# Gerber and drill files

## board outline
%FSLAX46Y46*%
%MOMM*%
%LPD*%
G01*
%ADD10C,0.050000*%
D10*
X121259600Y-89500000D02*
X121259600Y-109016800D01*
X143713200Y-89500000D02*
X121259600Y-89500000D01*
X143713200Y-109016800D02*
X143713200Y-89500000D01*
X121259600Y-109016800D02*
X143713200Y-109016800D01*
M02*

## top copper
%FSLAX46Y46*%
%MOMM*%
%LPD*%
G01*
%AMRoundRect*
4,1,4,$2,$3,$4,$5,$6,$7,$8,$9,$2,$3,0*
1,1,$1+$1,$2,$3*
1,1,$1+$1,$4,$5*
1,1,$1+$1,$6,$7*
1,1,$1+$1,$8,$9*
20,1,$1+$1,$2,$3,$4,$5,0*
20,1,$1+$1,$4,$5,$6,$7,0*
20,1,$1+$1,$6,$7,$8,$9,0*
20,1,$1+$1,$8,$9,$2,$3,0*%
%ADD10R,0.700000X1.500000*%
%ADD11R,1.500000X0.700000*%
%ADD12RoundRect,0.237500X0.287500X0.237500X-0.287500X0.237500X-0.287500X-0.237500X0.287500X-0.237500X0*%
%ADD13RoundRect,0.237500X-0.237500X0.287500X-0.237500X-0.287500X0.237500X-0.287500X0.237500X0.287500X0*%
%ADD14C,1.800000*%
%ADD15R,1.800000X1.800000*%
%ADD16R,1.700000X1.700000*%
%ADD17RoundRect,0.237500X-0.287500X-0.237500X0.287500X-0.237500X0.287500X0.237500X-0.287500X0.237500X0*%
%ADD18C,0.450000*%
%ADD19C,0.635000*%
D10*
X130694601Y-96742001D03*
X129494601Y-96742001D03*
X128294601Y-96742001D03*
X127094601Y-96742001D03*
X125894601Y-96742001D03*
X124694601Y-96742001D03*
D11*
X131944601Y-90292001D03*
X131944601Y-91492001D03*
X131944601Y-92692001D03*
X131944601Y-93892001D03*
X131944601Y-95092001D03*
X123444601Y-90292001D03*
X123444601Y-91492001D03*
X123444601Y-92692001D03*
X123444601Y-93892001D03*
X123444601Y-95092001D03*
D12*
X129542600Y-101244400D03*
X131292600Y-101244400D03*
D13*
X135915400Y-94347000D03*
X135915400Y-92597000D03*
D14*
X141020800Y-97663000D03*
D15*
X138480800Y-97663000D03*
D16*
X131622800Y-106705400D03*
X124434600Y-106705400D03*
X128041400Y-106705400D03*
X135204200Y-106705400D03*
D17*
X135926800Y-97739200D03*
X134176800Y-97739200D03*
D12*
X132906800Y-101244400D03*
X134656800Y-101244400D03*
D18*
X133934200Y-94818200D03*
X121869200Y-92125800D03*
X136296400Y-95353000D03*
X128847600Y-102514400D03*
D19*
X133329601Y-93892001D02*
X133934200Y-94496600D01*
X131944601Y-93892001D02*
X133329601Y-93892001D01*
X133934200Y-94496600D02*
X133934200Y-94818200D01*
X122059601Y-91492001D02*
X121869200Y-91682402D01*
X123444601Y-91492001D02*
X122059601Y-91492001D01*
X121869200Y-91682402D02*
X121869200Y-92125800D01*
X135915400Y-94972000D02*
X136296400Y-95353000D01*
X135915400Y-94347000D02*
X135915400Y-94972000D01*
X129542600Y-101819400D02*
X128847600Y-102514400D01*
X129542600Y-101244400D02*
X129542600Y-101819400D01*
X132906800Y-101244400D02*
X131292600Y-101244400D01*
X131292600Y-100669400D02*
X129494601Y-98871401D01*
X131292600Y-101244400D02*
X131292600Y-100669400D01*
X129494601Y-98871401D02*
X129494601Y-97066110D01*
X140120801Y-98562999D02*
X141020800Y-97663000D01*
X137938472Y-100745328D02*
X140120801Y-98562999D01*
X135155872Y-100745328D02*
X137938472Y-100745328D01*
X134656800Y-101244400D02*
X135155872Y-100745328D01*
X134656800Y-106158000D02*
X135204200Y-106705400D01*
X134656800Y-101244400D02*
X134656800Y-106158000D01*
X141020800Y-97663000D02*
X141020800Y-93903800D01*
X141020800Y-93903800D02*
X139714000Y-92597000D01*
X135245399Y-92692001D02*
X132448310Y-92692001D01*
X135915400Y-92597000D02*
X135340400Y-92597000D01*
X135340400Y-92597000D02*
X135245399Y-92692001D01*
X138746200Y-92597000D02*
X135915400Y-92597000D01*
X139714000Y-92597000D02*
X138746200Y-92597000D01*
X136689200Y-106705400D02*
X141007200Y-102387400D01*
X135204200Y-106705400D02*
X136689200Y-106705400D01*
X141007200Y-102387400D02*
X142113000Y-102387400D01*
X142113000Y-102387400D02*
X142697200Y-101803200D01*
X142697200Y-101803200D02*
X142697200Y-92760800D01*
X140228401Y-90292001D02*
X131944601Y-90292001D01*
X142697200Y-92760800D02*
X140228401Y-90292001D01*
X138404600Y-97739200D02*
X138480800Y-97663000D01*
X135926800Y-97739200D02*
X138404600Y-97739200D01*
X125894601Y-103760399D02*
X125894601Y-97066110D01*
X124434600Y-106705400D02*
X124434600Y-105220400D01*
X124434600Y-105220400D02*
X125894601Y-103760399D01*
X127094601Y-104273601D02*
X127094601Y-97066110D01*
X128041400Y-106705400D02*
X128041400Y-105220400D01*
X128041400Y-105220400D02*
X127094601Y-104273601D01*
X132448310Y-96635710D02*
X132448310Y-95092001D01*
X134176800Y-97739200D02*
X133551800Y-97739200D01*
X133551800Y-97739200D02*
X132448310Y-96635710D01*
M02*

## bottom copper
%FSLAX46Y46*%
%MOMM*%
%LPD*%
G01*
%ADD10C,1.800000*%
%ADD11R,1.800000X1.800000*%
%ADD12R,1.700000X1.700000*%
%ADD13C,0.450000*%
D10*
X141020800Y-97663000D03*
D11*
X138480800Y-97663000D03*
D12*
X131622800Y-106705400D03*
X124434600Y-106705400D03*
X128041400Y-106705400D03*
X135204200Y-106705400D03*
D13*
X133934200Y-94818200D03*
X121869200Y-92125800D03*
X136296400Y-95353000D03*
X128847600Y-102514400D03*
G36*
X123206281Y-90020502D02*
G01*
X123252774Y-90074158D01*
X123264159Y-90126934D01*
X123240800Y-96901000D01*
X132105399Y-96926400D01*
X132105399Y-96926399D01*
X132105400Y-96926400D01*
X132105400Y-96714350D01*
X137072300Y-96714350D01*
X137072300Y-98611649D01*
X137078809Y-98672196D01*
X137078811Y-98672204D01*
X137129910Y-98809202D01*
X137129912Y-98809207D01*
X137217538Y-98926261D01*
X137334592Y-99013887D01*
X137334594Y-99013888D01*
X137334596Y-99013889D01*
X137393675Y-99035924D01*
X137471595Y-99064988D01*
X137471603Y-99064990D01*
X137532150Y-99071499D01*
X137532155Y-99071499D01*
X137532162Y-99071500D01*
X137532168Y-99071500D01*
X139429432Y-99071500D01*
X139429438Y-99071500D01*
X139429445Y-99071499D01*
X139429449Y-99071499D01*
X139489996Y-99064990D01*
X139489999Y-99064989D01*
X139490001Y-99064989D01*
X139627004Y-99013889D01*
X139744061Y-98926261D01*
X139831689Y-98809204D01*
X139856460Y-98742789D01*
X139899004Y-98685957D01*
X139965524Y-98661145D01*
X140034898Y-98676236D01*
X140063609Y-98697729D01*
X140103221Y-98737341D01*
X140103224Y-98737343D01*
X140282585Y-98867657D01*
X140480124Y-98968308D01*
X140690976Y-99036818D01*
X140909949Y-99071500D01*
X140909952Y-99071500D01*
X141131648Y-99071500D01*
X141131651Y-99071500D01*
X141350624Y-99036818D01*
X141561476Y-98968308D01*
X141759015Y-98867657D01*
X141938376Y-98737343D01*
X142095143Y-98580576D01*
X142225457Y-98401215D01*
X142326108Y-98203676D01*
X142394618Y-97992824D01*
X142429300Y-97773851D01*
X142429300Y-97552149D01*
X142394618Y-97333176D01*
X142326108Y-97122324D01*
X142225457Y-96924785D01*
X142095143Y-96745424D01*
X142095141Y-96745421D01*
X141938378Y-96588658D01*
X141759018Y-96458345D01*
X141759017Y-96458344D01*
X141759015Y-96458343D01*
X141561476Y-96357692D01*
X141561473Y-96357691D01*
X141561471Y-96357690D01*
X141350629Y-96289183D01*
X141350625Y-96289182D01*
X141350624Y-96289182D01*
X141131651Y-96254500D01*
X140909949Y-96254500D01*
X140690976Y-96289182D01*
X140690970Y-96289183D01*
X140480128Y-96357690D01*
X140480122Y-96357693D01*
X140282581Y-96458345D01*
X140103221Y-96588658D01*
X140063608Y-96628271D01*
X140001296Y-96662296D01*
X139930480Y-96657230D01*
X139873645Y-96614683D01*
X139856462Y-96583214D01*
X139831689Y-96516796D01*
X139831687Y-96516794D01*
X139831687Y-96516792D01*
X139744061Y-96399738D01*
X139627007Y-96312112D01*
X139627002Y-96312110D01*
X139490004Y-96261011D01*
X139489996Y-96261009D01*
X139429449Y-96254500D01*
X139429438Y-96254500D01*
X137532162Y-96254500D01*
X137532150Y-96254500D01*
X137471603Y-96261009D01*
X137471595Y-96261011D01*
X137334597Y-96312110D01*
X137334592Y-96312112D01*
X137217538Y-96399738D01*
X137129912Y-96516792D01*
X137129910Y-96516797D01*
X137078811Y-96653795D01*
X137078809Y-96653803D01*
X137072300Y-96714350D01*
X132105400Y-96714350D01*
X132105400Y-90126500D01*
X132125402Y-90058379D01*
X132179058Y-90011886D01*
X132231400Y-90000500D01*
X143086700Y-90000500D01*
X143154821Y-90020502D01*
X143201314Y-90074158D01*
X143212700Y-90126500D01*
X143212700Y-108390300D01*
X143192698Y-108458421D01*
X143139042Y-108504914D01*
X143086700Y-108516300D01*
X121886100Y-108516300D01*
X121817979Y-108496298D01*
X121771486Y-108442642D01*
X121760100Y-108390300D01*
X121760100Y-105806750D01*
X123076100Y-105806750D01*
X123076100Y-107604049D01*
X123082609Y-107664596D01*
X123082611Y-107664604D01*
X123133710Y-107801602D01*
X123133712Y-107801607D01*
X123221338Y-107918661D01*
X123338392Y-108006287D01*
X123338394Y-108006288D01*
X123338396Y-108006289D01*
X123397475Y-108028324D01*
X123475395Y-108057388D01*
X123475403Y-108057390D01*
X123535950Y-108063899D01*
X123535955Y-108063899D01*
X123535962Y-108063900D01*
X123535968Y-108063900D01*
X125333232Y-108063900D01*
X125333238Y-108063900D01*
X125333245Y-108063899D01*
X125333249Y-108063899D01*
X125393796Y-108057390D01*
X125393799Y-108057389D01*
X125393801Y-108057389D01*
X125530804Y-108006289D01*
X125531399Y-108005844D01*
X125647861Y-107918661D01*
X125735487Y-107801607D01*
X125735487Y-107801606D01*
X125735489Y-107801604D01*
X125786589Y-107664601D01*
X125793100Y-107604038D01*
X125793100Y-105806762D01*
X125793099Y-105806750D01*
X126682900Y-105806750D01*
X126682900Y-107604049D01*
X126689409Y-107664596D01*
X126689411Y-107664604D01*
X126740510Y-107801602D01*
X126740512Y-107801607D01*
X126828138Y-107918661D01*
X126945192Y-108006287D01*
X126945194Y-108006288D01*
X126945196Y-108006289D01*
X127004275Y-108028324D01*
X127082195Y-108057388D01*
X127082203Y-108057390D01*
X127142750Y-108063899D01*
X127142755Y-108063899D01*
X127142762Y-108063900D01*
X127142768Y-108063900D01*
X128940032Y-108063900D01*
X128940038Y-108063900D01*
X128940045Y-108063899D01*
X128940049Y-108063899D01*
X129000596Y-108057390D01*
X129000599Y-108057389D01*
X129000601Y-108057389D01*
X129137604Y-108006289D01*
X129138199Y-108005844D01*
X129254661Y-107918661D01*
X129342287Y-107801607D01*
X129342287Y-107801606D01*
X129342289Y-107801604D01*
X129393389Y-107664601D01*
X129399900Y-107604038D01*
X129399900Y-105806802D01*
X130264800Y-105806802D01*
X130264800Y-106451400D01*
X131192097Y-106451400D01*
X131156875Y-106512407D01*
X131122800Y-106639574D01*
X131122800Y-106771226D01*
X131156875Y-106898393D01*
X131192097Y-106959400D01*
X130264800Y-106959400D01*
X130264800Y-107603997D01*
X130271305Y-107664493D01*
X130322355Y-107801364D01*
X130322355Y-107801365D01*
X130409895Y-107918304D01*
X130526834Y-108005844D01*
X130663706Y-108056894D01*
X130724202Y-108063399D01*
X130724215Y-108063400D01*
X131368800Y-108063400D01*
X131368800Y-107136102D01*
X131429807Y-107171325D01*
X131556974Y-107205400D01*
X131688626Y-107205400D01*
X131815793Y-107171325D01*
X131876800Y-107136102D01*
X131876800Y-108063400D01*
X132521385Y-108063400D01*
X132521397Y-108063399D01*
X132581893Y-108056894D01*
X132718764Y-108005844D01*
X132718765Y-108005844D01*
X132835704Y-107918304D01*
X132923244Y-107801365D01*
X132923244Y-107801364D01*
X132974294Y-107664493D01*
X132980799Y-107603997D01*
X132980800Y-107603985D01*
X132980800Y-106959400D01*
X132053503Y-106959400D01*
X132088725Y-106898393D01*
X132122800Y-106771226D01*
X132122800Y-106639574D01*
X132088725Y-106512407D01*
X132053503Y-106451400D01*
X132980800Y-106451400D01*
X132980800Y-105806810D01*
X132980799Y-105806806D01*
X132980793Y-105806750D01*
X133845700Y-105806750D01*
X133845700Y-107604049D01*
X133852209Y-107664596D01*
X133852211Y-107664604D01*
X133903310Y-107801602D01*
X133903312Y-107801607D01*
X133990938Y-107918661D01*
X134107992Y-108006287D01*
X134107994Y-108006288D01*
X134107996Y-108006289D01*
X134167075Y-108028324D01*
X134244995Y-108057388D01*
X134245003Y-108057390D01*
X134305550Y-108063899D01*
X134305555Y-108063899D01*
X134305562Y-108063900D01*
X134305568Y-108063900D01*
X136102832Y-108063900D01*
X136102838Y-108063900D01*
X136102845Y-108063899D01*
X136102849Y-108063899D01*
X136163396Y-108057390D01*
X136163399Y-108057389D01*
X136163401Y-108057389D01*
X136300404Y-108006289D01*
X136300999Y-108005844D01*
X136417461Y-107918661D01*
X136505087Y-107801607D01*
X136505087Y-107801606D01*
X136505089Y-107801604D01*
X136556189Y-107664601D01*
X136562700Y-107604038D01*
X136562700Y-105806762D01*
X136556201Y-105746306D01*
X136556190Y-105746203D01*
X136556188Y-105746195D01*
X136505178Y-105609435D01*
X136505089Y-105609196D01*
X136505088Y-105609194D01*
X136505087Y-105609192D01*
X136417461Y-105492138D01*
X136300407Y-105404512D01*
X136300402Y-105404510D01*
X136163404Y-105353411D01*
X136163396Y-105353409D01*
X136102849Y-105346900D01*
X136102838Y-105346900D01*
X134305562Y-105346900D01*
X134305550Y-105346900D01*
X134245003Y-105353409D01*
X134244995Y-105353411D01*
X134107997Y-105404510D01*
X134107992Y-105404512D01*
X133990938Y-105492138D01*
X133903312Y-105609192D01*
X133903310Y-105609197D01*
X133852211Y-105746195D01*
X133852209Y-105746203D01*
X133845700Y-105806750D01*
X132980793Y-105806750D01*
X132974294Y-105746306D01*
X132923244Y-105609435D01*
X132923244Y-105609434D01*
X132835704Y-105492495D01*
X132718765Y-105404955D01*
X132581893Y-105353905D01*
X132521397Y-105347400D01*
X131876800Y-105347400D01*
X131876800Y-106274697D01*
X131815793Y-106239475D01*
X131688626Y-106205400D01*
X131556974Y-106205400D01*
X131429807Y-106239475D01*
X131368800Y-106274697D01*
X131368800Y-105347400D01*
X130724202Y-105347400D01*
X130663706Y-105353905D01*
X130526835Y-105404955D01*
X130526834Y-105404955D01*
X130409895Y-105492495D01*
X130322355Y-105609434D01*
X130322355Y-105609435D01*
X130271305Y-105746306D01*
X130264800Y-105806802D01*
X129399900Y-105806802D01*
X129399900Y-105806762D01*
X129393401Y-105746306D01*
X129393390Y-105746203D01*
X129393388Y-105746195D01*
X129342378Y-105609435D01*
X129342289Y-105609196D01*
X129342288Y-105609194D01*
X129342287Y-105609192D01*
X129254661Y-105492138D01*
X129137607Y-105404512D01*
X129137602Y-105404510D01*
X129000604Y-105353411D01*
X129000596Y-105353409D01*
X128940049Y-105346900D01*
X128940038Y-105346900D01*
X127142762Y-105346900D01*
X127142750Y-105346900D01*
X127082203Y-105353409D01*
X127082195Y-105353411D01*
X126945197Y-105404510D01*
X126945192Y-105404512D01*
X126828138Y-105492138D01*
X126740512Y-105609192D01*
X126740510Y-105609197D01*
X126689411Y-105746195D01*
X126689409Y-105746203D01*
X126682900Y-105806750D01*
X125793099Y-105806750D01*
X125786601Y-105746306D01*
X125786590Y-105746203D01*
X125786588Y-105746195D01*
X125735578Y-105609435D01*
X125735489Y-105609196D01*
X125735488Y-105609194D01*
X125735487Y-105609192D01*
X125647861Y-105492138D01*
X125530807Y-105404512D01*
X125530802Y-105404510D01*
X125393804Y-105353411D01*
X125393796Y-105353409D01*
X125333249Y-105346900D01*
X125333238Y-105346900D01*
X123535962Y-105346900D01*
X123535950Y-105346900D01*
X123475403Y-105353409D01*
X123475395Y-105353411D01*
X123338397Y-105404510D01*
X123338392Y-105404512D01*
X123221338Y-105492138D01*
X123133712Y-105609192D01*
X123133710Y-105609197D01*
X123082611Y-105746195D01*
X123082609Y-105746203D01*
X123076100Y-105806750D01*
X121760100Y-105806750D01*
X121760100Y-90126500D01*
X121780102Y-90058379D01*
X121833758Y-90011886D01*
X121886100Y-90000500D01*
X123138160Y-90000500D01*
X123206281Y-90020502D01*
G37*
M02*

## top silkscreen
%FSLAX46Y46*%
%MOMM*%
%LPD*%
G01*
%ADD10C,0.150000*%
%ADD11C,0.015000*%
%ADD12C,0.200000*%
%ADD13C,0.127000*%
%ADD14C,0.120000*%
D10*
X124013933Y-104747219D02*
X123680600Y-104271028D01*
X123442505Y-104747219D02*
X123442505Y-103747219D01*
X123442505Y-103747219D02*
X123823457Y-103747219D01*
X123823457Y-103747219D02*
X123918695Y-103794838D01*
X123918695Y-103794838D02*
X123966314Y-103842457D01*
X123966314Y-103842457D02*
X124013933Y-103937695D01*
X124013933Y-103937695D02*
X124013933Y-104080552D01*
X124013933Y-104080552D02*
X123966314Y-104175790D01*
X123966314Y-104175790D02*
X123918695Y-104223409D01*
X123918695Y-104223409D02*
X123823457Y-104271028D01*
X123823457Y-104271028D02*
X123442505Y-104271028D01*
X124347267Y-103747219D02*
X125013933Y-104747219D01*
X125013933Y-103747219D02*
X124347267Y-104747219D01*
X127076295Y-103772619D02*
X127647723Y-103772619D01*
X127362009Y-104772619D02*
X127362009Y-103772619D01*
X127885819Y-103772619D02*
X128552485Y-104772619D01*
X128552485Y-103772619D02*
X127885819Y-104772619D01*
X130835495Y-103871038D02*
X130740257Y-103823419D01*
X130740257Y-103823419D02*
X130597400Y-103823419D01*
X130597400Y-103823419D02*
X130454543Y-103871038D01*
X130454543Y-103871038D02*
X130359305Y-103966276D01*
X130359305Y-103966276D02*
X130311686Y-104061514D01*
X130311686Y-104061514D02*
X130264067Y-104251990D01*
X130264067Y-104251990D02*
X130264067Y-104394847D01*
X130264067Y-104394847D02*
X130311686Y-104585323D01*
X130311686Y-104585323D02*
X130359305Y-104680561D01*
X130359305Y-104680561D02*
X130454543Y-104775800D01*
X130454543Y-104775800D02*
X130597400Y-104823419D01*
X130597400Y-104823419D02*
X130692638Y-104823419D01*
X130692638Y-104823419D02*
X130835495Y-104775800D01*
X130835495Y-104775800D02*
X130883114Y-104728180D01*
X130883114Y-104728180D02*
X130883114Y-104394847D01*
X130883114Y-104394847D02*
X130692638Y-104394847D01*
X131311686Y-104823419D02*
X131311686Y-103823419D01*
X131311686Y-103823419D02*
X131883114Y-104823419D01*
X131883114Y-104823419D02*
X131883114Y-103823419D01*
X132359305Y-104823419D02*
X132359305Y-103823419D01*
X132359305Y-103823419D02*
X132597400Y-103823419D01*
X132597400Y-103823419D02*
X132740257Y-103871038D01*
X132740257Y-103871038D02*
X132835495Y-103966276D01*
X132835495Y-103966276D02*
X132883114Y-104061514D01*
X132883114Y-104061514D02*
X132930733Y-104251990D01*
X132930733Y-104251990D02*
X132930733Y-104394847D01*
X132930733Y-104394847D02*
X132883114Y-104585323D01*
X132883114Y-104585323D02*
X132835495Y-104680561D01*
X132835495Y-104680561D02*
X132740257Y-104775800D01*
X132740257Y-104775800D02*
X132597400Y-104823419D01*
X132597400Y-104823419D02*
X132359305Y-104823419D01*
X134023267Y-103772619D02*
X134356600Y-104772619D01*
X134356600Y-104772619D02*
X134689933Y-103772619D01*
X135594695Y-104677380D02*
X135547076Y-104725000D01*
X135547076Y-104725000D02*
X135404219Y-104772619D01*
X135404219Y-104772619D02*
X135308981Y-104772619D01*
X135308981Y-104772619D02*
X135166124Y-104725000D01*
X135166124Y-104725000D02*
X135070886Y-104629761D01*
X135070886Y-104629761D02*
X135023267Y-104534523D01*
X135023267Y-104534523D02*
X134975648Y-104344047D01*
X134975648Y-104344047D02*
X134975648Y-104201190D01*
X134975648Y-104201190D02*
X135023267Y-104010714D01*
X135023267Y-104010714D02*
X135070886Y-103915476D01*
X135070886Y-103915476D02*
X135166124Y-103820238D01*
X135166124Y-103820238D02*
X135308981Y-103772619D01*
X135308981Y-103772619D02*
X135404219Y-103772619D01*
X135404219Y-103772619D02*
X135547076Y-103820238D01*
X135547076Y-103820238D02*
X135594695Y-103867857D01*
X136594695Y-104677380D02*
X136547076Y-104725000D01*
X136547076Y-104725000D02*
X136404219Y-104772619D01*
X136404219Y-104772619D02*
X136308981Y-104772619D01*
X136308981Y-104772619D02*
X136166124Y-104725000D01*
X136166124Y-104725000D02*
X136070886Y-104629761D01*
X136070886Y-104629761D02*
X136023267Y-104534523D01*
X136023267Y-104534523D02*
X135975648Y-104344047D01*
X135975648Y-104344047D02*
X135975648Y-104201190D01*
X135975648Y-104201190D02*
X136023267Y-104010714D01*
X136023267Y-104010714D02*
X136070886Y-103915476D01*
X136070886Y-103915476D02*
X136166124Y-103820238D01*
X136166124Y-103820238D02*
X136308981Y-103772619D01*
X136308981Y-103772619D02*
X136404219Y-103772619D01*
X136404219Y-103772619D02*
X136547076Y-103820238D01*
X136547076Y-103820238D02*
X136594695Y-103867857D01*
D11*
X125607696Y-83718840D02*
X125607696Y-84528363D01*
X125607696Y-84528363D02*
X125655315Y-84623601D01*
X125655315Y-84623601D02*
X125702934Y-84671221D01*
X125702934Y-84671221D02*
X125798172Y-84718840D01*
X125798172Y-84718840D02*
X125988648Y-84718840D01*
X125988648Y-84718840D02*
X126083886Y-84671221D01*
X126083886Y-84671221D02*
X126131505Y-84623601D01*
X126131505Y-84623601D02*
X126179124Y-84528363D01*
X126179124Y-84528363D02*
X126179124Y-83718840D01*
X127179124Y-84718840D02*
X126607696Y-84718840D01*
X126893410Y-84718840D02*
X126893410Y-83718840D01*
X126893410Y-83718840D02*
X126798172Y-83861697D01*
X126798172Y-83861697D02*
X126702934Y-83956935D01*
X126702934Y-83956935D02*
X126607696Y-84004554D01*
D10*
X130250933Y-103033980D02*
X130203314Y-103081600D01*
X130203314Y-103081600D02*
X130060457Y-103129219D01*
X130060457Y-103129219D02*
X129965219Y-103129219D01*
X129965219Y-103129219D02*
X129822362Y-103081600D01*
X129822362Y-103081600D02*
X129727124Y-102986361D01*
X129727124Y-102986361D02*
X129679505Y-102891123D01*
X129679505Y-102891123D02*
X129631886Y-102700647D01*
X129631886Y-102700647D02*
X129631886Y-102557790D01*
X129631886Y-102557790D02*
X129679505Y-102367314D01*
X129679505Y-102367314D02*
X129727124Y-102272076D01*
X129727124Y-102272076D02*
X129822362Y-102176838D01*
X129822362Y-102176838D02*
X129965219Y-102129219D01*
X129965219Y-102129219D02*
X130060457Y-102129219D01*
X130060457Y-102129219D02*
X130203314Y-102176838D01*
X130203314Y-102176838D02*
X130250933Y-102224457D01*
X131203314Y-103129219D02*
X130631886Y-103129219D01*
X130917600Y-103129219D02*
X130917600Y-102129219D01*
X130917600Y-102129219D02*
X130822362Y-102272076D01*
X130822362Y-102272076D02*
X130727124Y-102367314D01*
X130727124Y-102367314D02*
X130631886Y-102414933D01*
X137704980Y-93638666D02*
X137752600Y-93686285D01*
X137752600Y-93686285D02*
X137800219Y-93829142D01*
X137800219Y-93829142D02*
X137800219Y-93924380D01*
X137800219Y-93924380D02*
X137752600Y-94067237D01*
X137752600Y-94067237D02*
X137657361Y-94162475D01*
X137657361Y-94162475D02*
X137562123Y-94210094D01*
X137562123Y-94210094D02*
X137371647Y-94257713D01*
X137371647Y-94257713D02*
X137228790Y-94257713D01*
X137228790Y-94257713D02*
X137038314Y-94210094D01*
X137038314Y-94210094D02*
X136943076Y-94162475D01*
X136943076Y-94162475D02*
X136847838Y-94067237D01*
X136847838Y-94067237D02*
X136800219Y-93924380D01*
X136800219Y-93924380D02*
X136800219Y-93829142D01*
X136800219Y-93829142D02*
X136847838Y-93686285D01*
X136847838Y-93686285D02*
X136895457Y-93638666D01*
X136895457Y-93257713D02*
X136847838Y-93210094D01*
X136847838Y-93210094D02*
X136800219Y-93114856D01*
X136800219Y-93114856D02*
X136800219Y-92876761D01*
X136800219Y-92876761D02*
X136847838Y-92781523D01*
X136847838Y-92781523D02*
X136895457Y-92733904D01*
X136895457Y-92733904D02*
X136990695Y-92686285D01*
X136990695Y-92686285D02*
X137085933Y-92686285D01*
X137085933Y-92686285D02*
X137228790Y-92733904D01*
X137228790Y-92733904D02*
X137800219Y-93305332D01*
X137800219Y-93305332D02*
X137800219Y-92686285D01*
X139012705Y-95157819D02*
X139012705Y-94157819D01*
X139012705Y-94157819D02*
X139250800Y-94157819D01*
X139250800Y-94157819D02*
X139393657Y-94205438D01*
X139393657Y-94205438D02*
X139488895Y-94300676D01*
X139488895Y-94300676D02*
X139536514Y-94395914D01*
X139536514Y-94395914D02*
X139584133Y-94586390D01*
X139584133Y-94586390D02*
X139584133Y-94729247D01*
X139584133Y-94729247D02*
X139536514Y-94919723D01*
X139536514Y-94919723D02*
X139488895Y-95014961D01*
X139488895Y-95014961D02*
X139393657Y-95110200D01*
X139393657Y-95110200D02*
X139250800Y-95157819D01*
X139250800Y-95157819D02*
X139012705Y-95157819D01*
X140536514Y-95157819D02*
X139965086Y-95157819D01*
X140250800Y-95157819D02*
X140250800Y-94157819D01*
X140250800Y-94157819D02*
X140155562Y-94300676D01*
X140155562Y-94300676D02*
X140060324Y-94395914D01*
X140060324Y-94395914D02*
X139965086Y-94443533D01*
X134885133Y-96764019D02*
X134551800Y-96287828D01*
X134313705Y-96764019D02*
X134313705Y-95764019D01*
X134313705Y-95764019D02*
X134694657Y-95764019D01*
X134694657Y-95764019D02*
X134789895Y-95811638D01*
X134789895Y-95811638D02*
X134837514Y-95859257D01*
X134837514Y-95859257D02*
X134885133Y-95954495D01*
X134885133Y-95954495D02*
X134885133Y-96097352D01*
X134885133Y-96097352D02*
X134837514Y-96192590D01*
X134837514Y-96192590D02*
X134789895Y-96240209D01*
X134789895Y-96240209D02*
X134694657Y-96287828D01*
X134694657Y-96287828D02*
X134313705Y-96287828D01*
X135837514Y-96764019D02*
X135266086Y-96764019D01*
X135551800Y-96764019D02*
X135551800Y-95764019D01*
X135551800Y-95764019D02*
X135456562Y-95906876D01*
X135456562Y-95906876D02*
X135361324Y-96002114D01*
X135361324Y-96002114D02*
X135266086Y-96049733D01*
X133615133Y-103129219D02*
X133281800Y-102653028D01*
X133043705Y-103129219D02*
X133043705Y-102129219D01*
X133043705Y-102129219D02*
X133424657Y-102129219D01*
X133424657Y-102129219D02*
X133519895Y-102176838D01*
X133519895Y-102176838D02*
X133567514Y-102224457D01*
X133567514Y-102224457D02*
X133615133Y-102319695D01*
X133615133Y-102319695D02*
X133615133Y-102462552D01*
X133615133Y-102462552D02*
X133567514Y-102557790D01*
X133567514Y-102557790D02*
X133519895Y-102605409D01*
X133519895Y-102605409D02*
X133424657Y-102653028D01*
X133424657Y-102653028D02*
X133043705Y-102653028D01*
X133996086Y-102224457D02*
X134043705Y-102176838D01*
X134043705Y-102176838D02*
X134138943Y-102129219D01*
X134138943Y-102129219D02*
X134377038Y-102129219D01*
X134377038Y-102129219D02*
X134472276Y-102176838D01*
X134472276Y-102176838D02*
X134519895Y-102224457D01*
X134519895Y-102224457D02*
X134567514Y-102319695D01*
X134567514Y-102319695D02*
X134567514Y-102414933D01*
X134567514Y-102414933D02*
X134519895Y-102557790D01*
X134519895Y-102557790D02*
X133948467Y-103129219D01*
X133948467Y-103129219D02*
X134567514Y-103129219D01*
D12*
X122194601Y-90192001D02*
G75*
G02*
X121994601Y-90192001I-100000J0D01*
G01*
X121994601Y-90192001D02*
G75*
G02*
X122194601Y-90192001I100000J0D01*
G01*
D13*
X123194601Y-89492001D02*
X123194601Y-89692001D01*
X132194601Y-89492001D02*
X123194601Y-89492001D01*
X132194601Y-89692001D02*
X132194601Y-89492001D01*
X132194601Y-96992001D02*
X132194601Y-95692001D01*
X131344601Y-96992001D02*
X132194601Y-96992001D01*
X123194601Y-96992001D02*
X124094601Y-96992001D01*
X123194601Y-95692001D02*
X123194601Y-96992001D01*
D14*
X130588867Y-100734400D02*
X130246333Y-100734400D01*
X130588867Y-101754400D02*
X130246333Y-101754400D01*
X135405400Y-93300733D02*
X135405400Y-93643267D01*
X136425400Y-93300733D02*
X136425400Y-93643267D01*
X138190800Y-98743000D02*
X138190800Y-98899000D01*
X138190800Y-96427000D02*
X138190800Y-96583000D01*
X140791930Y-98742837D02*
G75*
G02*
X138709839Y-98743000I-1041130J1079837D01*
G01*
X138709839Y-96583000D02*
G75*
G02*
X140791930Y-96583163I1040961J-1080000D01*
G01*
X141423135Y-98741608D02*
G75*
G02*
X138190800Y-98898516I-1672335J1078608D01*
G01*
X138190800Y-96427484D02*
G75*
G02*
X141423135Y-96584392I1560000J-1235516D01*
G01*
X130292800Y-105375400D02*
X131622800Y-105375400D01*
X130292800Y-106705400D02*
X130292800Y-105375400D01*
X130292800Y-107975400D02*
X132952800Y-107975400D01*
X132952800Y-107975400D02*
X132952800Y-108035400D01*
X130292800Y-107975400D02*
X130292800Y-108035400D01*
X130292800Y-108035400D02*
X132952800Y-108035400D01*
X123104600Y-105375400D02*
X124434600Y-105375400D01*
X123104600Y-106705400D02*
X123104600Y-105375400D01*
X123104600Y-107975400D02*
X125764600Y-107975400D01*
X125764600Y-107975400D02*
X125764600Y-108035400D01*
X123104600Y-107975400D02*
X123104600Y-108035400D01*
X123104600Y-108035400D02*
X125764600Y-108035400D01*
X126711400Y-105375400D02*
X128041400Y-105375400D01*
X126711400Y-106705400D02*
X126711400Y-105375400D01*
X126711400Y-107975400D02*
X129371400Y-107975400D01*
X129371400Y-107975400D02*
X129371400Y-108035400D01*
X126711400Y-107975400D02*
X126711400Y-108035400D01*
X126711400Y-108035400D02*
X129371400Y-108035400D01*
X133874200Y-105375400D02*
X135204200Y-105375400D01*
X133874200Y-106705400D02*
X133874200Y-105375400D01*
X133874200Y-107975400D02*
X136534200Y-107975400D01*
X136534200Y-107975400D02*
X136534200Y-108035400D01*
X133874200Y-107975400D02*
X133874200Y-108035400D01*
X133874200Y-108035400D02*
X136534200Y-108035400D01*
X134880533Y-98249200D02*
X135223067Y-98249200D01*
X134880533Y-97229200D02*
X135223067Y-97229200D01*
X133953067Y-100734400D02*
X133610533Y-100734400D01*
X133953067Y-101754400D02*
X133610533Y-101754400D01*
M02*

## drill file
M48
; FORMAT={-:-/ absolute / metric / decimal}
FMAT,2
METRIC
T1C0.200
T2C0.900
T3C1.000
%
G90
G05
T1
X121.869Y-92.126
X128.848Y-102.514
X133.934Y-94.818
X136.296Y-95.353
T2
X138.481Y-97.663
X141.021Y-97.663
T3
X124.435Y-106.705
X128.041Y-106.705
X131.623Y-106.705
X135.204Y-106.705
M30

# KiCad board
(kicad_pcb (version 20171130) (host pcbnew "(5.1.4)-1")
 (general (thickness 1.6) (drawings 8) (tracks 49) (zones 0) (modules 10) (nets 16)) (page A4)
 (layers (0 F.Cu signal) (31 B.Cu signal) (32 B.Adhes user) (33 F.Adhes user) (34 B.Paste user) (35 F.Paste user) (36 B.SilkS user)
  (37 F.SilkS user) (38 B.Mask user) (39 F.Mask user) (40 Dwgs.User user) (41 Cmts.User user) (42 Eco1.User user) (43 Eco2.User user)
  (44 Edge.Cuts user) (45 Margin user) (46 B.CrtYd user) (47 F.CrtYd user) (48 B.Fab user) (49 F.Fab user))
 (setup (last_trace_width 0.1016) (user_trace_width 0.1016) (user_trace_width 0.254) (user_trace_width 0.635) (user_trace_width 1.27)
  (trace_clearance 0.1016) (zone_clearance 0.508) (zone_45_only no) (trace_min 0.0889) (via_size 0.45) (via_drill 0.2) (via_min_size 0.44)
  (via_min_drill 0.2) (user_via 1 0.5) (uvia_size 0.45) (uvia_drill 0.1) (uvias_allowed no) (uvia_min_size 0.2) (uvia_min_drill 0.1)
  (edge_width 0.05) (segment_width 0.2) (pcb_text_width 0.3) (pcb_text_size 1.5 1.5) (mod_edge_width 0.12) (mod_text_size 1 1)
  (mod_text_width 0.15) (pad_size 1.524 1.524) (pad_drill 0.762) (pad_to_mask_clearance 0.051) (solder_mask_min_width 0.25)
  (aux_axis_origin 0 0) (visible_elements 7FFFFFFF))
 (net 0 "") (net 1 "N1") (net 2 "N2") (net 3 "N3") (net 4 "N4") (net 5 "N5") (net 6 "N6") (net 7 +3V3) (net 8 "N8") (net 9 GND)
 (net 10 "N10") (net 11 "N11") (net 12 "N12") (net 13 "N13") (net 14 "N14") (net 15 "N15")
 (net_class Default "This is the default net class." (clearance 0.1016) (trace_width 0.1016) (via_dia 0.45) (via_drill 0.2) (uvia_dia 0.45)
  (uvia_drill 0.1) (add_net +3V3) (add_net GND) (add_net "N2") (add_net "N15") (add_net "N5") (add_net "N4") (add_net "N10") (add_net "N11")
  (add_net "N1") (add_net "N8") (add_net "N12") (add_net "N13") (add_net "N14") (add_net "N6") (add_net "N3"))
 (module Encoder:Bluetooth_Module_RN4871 (layer F.Cu) (at 127.694601 91.242001)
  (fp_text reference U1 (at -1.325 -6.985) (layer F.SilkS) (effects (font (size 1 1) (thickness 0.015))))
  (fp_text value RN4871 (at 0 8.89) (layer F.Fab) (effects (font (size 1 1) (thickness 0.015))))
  (fp_circle (center -5.6 -1.05) (end -5.5 -1.05) (layer F.SilkS) (width 0.2))
  (fp_line (start -4.5 -1.75) (end -4.5 -1.55) (layer F.SilkS) (width 0.127))
  (fp_line (start 4.5 -1.75) (end -4.5 -1.75) (layer F.SilkS) (width 0.127))
  (fp_line (start 4.5 -1.55) (end 4.5 -1.75) (layer F.SilkS) (width 0.127))
  (fp_line (start 4.5 5.75) (end 4.5 4.45) (layer F.SilkS) (width 0.127))
  (fp_line (start 3.65 5.75) (end 4.5 5.75) (layer F.SilkS) (width 0.127))
  (fp_line (start -4.5 5.75) (end -3.6 5.75) (layer F.SilkS) (width 0.127))
  (fp_line (start -4.5 4.45) (end -4.5 5.75) (layer F.SilkS) (width 0.127))
  (pad 11 smd rect (at 3 5.5) (size 0.7 1.5) (layers F.Cu F.Paste F.Mask) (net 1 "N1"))
  (pad 10 smd rect (at 1.8 5.5) (size 0.7 1.5) (layers F.Cu F.Paste F.Mask) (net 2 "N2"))
  (pad 9 smd rect (at 0.6 5.5) (size 0.7 1.5) (layers F.Cu F.Paste F.Mask) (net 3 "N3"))
  (pad 8 smd rect (at -0.6 5.5) (size 0.7 1.5) (layers F.Cu F.Paste F.Mask) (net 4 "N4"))
  (pad 7 smd rect (at -1.8 5.5) (size 0.7 1.5) (layers F.Cu F.Paste F.Mask) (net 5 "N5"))
  (pad 6 smd rect (at -3 5.5) (size 0.7 1.5) (layers F.Cu F.Paste F.Mask) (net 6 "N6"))
  (pad 16 smd rect (at 4.25 -0.95) (size 1.5 0.7) (layers F.Cu F.Paste F.Mask) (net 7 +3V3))
  (pad 15 smd rect (at 4.25 0.25) (size 1.5 0.7) (layers F.Cu F.Paste F.Mask) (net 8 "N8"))
  (pad 14 smd rect (at 4.25 1.45) (size 1.5 0.7) (layers F.Cu F.Paste F.Mask) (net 7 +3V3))
  (pad 13 smd rect (at 4.25 2.65) (size 1.5 0.7) (layers F.Cu F.Paste F.Mask) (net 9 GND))
  (pad 12 smd rect (at 4.25 3.85) (size 1.5 0.7) (layers F.Cu F.Paste F.Mask) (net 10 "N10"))
  (pad 1 smd rect (at -4.25 -0.95) (size 1.5 0.7) (layers F.Cu F.Paste F.Mask) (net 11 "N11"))
  (pad 2 smd rect (at -4.25 0.25) (size 1.5 0.7) (layers F.Cu F.Paste F.Mask) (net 9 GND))
  (pad 3 smd rect (at -4.25 1.45) (size 1.5 0.7) (layers F.Cu F.Paste F.Mask) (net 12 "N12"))
  (pad 4 smd rect (at -4.25 2.65) (size 1.5 0.7) (layers F.Cu F.Paste F.Mask) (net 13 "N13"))
  (pad 5 smd rect (at -4.25 3.85) (size 1.5 0.7) (layers F.Cu F.Paste F.Mask) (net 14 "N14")))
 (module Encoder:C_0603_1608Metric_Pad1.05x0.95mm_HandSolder (layer F.Cu) (at 130.4176 101.2444 180)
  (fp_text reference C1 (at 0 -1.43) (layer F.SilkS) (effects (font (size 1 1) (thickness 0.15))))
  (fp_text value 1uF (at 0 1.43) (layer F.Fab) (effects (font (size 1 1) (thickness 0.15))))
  (fp_line (start -0.171267 0.51) (end 0.171267 0.51) (layer F.SilkS) (width 0.12))
  (fp_line (start -0.171267 -0.51) (end 0.171267 -0.51) (layer F.SilkS) (width 0.12))
  (pad 2 smd roundrect (at 0.875 0 180) (size 1.05 0.95) (layers F.Cu F.Paste F.Mask) (roundrect_rratio 0.25) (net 9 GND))
  (pad 1 smd roundrect (at -0.875 0 180) (size 1.05 0.95) (layers F.Cu F.Paste F.Mask) (roundrect_rratio 0.25) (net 2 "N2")))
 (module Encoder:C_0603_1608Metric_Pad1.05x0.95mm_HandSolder (layer F.Cu) (at 135.9154 93.472 270)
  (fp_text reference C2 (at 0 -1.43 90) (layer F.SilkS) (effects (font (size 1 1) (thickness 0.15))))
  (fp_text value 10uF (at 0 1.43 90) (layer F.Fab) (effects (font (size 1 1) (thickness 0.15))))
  (fp_line (start -0.171267 0.51) (end 0.171267 0.51) (layer F.SilkS) (width 0.12))
  (fp_line (start -0.171267 -0.51) (end 0.171267 -0.51) (layer F.SilkS) (width 0.12))
  (pad 2 smd roundrect (at 0.875 0 270) (size 1.05 0.95) (layers F.Cu F.Paste F.Mask) (roundrect_rratio 0.25) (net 9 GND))
  (pad 1 smd roundrect (at -0.875 0 270) (size 1.05 0.95) (layers F.Cu F.Paste F.Mask) (roundrect_rratio 0.25) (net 7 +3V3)))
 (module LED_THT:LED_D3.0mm (layer F.Cu) (at 138.4808 97.663)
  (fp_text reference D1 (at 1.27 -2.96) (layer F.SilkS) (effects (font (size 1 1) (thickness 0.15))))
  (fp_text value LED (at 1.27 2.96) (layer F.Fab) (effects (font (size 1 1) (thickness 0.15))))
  (fp_line (start -0.29 1.08) (end -0.29 1.236) (layer F.SilkS) (width 0.12))
  (fp_line (start -0.29 -1.236) (end -0.29 -1.08) (layer F.SilkS) (width 0.12))
  (fp_arc (start 1.27 0) (end 0.229039 1.08) (angle -87.9) (layer F.SilkS) (width 0.12))
  (fp_arc (start 1.27 0) (end 0.229039 -1.08) (angle 87.9) (layer F.SilkS) (width 0.12))
  (fp_arc (start 1.27 0) (end -0.29 1.235516) (angle -108.8) (layer F.SilkS) (width 0.12))
  (fp_arc (start 1.27 0) (end -0.29 -1.235516) (angle 108.8) (layer F.SilkS) (width 0.12))
  (pad 2 thru_hole circle (at 2.54 0) (size 1.8 1.8) (drill 0.9) (layers *.Cu *.Mask) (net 7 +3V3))
  (pad 1 thru_hole rect (at 0 0) (size 1.8 1.8) (drill 0.9) (layers *.Cu *.Mask) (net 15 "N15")))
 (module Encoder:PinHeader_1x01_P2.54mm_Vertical (layer F.Cu) (at 131.6228 106.7054)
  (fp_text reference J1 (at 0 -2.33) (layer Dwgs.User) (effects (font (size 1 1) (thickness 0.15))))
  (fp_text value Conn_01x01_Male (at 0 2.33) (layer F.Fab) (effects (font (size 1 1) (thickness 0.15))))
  (fp_line (start -1.33 -1.33) (end 0 -1.33) (layer F.SilkS) (width 0.12))
  (fp_line (start -1.33 0) (end -1.33 -1.33) (layer F.SilkS) (width 0.12))
  (fp_line (start -1.33 1.27) (end 1.33 1.27) (layer F.SilkS) (width 0.12))
  (fp_line (start 1.33 1.27) (end 1.33 1.33) (layer F.SilkS) (width 0.12))
  (fp_line (start -1.33 1.27) (end -1.33 1.33) (layer F.SilkS) (width 0.12))
  (fp_line (start -1.33 1.33) (end 1.33 1.33) (layer F.SilkS) (width 0.12))
  (pad 1 thru_hole rect (at 0 0) (size 1.7 1.7) (drill 1) (layers *.Cu *.Mask) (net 9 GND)))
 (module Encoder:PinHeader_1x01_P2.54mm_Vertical (layer F.Cu) (at 124.4346 106.7054)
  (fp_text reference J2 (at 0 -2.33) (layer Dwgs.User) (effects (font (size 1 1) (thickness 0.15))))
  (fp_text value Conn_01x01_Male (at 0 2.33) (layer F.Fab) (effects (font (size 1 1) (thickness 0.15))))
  (fp_line (start -1.33 -1.33) (end 0 -1.33) (layer F.SilkS) (width 0.12))
  (fp_line (start -1.33 0) (end -1.33 -1.33) (layer F.SilkS) (width 0.12))
  (fp_line (start -1.33 1.27) (end 1.33 1.27) (layer F.SilkS) (width 0.12))
  (fp_line (start 1.33 1.27) (end 1.33 1.33) (layer F.SilkS) (width 0.12))
  (fp_line (start -1.33 1.27) (end -1.33 1.33) (layer F.SilkS) (width 0.12))
  (fp_line (start -1.33 1.33) (end 1.33 1.33) (layer F.SilkS) (width 0.12))
  (pad 1 thru_hole rect (at 0 0) (size 1.7 1.7) (drill 1) (layers *.Cu *.Mask) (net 5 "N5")))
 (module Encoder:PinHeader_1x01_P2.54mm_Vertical (layer F.Cu) (at 128.0414 106.7054)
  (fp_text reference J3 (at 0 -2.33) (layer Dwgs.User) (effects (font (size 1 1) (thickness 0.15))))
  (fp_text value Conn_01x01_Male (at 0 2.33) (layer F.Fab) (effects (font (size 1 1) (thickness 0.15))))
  (fp_line (start -1.33 -1.33) (end 0 -1.33) (layer F.SilkS) (width 0.12))
  (fp_line (start -1.33 0) (end -1.33 -1.33) (layer F.SilkS) (width 0.12))
  (fp_line (start -1.33 1.27) (end 1.33 1.27) (layer F.SilkS) (width 0.12))
  (fp_line (start 1.33 1.27) (end 1.33 1.33) (layer F.SilkS) (width 0.12))
  (fp_line (start -1.33 1.27) (end -1.33 1.33) (layer F.SilkS) (width 0.12))
  (fp_line (start -1.33 1.33) (end 1.33 1.33) (layer F.SilkS) (width 0.12))
  (pad 1 thru_hole rect (at 0 0) (size 1.7 1.7) (drill 1) (layers *.Cu *.Mask) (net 4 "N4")))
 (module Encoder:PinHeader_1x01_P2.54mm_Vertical (layer F.Cu) (at 135.2042 106.7054)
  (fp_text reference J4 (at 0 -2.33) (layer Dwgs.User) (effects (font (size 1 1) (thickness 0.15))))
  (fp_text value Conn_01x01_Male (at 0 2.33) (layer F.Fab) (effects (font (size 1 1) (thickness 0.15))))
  (fp_line (start -1.33 -1.33) (end 0 -1.33) (layer F.SilkS) (width 0.12))
  (fp_line (start -1.33 0) (end -1.33 -1.33) (layer F.SilkS) (width 0.12))
  (fp_line (start -1.33 1.27) (end 1.33 1.27) (layer F.SilkS) (width 0.12))
  (fp_line (start 1.33 1.27) (end 1.33 1.33) (layer F.SilkS) (width 0.12))
  (fp_line (start -1.33 1.27) (end -1.33 1.33) (layer F.SilkS) (width 0.12))
  (fp_line (start -1.33 1.33) (end 1.33 1.33) (layer F.SilkS) (width 0.12))
  (pad 1 thru_hole rect (at 0 0) (size 1.7 1.7) (drill 1) (layers *.Cu *.Mask) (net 7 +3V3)))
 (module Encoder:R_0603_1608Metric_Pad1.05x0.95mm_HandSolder (layer F.Cu) (at 135.0518 97.7392)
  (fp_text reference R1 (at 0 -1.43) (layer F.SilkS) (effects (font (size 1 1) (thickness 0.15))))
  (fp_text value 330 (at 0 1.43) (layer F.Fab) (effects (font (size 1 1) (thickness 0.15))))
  (fp_line (start -0.171267 0.51) (end 0.171267 0.51) (layer F.SilkS) (width 0.12))
  (fp_line (start -0.171267 -0.51) (end 0.171267 -0.51) (layer F.SilkS) (width 0.12))
  (pad 2 smd roundrect (at 0.875 0) (size 1.05 0.95) (layers F.Cu F.Paste F.Mask) (roundrect_rratio 0.25) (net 15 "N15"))
  (pad 1 smd roundrect (at -0.875 0) (size 1.05 0.95) (layers F.Cu F.Paste F.Mask) (roundrect_rratio 0.25) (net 10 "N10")))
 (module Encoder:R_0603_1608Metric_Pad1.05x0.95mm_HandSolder (layer F.Cu) (at 133.7818 101.2444 180)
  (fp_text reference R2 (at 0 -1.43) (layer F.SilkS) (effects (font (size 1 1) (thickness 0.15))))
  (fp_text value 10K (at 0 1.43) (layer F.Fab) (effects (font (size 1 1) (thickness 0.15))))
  (fp_line (start -0.171267 0.51) (end 0.171267 0.51) (layer F.SilkS) (width 0.12))
  (fp_line (start -0.171267 -0.51) (end 0.171267 -0.51) (layer F.SilkS) (width 0.12))
  (pad 2 smd roundrect (at 0.875 0 180) (size 1.05 0.95) (layers F.Cu F.Paste F.Mask) (roundrect_rratio 0.25) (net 2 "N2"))
  (pad 1 smd roundrect (at -0.875 0 180) (size 1.05 0.95) (layers F.Cu F.Paste F.Mask) (roundrect_rratio 0.25) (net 7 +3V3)))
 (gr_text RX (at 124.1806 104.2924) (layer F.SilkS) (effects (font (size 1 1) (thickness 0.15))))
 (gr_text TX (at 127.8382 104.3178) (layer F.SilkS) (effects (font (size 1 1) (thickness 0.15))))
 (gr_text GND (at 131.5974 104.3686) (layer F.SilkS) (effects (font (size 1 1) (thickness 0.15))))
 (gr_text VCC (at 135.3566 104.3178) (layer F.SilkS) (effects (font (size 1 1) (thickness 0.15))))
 (gr_line (start 121.2596 89.5) (end 121.2596 109.0168) (layer Edge.Cuts) (width 0.05))
 (gr_line (start 143.7132 89.5) (end 121.2596 89.5) (layer Edge.Cuts) (width 0.05))
 (gr_line (start 143.7132 109.0168) (end 143.7132 89.5) (layer Edge.Cuts) (width 0.05))
 (gr_line (start 121.2596 109.0168) (end 143.7132 109.0168) (layer Edge.Cuts) (width 0.05))
 (segment (start 133.329601 93.892001) (end 133.9342 94.4966) (width 0.635) (layer F.Cu) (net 9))
 (segment (start 131.944601 93.892001) (end 133.329601 93.892001) (width 0.635) (layer F.Cu) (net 9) (status 10))
 (segment (start 133.9342 94.4966) (end 133.9342 94.8182) (width 0.635) (layer F.Cu) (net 9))
 (via (at 133.9342 94.8182) (size 0.45) (drill 0.2) (layers F.Cu B.Cu) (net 9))
 (segment (start 122.059601 91.492001) (end 121.8692 91.682402) (width 0.635) (layer F.Cu) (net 9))
 (segment (start 123.444601 91.492001) (end 122.059601 91.492001) (width 0.635) (layer F.Cu) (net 9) (status 10))
 (segment (start 121.8692 91.682402) (end 121.8692 92.1258) (width 0.635) (layer F.Cu) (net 9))
 (via (at 121.8692 92.1258) (size 0.45) (drill 0.2) (layers F.Cu B.Cu) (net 9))
 (segment (start 135.9154 94.972) (end 136.2964 95.353) (width 0.635) (layer F.Cu) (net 9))
 (segment (start 135.9154 94.347) (end 135.9154 94.972) (width 0.635) (layer F.Cu) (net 9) (status 10))
 (via (at 136.2964 95.353) (size 0.45) (drill 0.2) (layers F.Cu B.Cu) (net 9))
 (segment (start 129.5426 101.8194) (end 128.8476 102.5144) (width 0.635) (layer F.Cu) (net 9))
 (segment (start 129.5426 101.2444) (end 129.5426 101.8194) (width 0.635) (layer F.Cu) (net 9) (status 10))
 (via (at 128.8476 102.5144) (size 0.45) (drill 0.2) (layers F.Cu B.Cu) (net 9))
 (segment (start 132.9068 101.2444) (end 131.2926 101.2444) (width 0.635) (layer F.Cu) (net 2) (status 30))
 (segment (start 131.2926 100.6694) (end 129.494601 98.871401) (width 0.635) (layer F.Cu) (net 2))
 (segment (start 131.2926 101.2444) (end 131.2926 100.6694) (width 0.635) (layer F.Cu) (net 2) (status 10))
 (segment (start 129.494601 98.871401) (end 129.494601 97.06611) (width 0.635) (layer F.Cu) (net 2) (status 20))
 (segment (start 140.120801 98.562999) (end 141.0208 97.663) (width 0.635) (layer F.Cu) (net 7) (status 20))
 (segment (start 137.938472 100.745328) (end 140.120801 98.562999) (width 0.635) (layer F.Cu) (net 7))
 (segment (start 135.155872 100.745328) (end 137.938472 100.745328) (width 0.635) (layer F.Cu) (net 7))
 (segment (start 134.6568 101.2444) (end 135.155872 100.745328) (width 0.635) (layer F.Cu) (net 7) (status 10))
 (segment (start 134.6568 106.158) (end 135.2042 106.7054) (width 0.635) (layer F.Cu) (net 7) (status 30))
 (segment (start 134.6568 101.2444) (end 134.6568 106.158) (width 0.635) (layer F.Cu) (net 7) (status 30))
 (segment (start 141.0208 97.663) (end 141.0208 93.9038) (width 0.635) (layer F.Cu) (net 7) (status 10))
 (segment (start 141.0208 93.9038) (end 139.714 92.597) (width 0.635) (layer F.Cu) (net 7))
 (segment (start 135.245399 92.692001) (end 132.44831 92.692001) (width 0.635) (layer F.Cu) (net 7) (status 20))
 (segment (start 135.9154 92.597) (end 135.3404 92.597) (width 0.635) (layer F.Cu) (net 7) (status 10))
 (segment (start 135.3404 92.597) (end 135.245399 92.692001) (width 0.635) (layer F.Cu) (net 7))
 (segment (start 138.7462 92.597) (end 135.9154 92.597) (width 0.635) (layer F.Cu) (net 7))
 (segment (start 139.714 92.597) (end 138.7462 92.597) (width 0.635) (layer F.Cu) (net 7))
 (segment (start 136.6892 106.7054) (end 141.0072 102.3874) (width 0.635) (layer F.Cu) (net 7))
 (segment (start 135.2042 106.7054) (end 136.6892 106.7054) (width 0.635) (layer F.Cu) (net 7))
 (segment (start 141.0072 102.3874) (end 142.113 102.3874) (width 0.635) (layer F.Cu) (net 7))
 (segment (start 142.113 102.3874) (end 142.6972 101.8032) (width 0.635) (layer F.Cu) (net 7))
 (segment (start 142.6972 101.8032) (end 142.6972 92.7608) (width 0.635) (layer F.Cu) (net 7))
 (segment (start 140.228401 90.292001) (end 131.944601 90.292001) (width 0.635) (layer F.Cu) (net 7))
 (segment (start 142.6972 92.7608) (end 140.228401 90.292001) (width 0.635) (layer F.Cu) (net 7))
 (segment (start 138.4046 97.7392) (end 138.4808 97.663) (width 0.635) (layer F.Cu) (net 15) (status 30))
 (segment (start 135.9268 97.7392) (end 138.4046 97.7392) (width 0.635) (layer F.Cu) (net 15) (status 30))
 (segment (start 125.894601 103.760399) (end 125.894601 97.06611) (width 0.635) (layer F.Cu) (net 5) (status 20))
 (segment (start 124.4346 106.7054) (end 124.4346 105.2204) (width 0.635) (layer F.Cu) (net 5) (status 10))
 (segment (start 124.4346 105.2204) (end 125.894601 103.760399) (width 0.635) (layer F.Cu) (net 5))
 (segment (start 127.094601 104.273601) (end 127.094601 97.06611) (width 0.635) (layer F.Cu) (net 4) (status 20))
 (segment (start 128.0414 106.7054) (end 128.0414 105.2204) (width 0.635) (layer F.Cu) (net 4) (status 10))
 (segment (start 128.0414 105.2204) (end 127.094601 104.273601) (width 0.635) (layer F.Cu) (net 4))
 (segment (start 132.44831 96.63571) (end 132.44831 95.092001) (width 0.635) (layer F.Cu) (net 10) (status 20))
 (segment (start 134.1768 97.7392) (end 133.5518 97.7392) (width 0.635) (layer F.Cu) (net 10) (status 10))
 (segment (start 133.5518 97.7392) (end 132.44831 96.63571) (width 0.635) (layer F.Cu) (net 10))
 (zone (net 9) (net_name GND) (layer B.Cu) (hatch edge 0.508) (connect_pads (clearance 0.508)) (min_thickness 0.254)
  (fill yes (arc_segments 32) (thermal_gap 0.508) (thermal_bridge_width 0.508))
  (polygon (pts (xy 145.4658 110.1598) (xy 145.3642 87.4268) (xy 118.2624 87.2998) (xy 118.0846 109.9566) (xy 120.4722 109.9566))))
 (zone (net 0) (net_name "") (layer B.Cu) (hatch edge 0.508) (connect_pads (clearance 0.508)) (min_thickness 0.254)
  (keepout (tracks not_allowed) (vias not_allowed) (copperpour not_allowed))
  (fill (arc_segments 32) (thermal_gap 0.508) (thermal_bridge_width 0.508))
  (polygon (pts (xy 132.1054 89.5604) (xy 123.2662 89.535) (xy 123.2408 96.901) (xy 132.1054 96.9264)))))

